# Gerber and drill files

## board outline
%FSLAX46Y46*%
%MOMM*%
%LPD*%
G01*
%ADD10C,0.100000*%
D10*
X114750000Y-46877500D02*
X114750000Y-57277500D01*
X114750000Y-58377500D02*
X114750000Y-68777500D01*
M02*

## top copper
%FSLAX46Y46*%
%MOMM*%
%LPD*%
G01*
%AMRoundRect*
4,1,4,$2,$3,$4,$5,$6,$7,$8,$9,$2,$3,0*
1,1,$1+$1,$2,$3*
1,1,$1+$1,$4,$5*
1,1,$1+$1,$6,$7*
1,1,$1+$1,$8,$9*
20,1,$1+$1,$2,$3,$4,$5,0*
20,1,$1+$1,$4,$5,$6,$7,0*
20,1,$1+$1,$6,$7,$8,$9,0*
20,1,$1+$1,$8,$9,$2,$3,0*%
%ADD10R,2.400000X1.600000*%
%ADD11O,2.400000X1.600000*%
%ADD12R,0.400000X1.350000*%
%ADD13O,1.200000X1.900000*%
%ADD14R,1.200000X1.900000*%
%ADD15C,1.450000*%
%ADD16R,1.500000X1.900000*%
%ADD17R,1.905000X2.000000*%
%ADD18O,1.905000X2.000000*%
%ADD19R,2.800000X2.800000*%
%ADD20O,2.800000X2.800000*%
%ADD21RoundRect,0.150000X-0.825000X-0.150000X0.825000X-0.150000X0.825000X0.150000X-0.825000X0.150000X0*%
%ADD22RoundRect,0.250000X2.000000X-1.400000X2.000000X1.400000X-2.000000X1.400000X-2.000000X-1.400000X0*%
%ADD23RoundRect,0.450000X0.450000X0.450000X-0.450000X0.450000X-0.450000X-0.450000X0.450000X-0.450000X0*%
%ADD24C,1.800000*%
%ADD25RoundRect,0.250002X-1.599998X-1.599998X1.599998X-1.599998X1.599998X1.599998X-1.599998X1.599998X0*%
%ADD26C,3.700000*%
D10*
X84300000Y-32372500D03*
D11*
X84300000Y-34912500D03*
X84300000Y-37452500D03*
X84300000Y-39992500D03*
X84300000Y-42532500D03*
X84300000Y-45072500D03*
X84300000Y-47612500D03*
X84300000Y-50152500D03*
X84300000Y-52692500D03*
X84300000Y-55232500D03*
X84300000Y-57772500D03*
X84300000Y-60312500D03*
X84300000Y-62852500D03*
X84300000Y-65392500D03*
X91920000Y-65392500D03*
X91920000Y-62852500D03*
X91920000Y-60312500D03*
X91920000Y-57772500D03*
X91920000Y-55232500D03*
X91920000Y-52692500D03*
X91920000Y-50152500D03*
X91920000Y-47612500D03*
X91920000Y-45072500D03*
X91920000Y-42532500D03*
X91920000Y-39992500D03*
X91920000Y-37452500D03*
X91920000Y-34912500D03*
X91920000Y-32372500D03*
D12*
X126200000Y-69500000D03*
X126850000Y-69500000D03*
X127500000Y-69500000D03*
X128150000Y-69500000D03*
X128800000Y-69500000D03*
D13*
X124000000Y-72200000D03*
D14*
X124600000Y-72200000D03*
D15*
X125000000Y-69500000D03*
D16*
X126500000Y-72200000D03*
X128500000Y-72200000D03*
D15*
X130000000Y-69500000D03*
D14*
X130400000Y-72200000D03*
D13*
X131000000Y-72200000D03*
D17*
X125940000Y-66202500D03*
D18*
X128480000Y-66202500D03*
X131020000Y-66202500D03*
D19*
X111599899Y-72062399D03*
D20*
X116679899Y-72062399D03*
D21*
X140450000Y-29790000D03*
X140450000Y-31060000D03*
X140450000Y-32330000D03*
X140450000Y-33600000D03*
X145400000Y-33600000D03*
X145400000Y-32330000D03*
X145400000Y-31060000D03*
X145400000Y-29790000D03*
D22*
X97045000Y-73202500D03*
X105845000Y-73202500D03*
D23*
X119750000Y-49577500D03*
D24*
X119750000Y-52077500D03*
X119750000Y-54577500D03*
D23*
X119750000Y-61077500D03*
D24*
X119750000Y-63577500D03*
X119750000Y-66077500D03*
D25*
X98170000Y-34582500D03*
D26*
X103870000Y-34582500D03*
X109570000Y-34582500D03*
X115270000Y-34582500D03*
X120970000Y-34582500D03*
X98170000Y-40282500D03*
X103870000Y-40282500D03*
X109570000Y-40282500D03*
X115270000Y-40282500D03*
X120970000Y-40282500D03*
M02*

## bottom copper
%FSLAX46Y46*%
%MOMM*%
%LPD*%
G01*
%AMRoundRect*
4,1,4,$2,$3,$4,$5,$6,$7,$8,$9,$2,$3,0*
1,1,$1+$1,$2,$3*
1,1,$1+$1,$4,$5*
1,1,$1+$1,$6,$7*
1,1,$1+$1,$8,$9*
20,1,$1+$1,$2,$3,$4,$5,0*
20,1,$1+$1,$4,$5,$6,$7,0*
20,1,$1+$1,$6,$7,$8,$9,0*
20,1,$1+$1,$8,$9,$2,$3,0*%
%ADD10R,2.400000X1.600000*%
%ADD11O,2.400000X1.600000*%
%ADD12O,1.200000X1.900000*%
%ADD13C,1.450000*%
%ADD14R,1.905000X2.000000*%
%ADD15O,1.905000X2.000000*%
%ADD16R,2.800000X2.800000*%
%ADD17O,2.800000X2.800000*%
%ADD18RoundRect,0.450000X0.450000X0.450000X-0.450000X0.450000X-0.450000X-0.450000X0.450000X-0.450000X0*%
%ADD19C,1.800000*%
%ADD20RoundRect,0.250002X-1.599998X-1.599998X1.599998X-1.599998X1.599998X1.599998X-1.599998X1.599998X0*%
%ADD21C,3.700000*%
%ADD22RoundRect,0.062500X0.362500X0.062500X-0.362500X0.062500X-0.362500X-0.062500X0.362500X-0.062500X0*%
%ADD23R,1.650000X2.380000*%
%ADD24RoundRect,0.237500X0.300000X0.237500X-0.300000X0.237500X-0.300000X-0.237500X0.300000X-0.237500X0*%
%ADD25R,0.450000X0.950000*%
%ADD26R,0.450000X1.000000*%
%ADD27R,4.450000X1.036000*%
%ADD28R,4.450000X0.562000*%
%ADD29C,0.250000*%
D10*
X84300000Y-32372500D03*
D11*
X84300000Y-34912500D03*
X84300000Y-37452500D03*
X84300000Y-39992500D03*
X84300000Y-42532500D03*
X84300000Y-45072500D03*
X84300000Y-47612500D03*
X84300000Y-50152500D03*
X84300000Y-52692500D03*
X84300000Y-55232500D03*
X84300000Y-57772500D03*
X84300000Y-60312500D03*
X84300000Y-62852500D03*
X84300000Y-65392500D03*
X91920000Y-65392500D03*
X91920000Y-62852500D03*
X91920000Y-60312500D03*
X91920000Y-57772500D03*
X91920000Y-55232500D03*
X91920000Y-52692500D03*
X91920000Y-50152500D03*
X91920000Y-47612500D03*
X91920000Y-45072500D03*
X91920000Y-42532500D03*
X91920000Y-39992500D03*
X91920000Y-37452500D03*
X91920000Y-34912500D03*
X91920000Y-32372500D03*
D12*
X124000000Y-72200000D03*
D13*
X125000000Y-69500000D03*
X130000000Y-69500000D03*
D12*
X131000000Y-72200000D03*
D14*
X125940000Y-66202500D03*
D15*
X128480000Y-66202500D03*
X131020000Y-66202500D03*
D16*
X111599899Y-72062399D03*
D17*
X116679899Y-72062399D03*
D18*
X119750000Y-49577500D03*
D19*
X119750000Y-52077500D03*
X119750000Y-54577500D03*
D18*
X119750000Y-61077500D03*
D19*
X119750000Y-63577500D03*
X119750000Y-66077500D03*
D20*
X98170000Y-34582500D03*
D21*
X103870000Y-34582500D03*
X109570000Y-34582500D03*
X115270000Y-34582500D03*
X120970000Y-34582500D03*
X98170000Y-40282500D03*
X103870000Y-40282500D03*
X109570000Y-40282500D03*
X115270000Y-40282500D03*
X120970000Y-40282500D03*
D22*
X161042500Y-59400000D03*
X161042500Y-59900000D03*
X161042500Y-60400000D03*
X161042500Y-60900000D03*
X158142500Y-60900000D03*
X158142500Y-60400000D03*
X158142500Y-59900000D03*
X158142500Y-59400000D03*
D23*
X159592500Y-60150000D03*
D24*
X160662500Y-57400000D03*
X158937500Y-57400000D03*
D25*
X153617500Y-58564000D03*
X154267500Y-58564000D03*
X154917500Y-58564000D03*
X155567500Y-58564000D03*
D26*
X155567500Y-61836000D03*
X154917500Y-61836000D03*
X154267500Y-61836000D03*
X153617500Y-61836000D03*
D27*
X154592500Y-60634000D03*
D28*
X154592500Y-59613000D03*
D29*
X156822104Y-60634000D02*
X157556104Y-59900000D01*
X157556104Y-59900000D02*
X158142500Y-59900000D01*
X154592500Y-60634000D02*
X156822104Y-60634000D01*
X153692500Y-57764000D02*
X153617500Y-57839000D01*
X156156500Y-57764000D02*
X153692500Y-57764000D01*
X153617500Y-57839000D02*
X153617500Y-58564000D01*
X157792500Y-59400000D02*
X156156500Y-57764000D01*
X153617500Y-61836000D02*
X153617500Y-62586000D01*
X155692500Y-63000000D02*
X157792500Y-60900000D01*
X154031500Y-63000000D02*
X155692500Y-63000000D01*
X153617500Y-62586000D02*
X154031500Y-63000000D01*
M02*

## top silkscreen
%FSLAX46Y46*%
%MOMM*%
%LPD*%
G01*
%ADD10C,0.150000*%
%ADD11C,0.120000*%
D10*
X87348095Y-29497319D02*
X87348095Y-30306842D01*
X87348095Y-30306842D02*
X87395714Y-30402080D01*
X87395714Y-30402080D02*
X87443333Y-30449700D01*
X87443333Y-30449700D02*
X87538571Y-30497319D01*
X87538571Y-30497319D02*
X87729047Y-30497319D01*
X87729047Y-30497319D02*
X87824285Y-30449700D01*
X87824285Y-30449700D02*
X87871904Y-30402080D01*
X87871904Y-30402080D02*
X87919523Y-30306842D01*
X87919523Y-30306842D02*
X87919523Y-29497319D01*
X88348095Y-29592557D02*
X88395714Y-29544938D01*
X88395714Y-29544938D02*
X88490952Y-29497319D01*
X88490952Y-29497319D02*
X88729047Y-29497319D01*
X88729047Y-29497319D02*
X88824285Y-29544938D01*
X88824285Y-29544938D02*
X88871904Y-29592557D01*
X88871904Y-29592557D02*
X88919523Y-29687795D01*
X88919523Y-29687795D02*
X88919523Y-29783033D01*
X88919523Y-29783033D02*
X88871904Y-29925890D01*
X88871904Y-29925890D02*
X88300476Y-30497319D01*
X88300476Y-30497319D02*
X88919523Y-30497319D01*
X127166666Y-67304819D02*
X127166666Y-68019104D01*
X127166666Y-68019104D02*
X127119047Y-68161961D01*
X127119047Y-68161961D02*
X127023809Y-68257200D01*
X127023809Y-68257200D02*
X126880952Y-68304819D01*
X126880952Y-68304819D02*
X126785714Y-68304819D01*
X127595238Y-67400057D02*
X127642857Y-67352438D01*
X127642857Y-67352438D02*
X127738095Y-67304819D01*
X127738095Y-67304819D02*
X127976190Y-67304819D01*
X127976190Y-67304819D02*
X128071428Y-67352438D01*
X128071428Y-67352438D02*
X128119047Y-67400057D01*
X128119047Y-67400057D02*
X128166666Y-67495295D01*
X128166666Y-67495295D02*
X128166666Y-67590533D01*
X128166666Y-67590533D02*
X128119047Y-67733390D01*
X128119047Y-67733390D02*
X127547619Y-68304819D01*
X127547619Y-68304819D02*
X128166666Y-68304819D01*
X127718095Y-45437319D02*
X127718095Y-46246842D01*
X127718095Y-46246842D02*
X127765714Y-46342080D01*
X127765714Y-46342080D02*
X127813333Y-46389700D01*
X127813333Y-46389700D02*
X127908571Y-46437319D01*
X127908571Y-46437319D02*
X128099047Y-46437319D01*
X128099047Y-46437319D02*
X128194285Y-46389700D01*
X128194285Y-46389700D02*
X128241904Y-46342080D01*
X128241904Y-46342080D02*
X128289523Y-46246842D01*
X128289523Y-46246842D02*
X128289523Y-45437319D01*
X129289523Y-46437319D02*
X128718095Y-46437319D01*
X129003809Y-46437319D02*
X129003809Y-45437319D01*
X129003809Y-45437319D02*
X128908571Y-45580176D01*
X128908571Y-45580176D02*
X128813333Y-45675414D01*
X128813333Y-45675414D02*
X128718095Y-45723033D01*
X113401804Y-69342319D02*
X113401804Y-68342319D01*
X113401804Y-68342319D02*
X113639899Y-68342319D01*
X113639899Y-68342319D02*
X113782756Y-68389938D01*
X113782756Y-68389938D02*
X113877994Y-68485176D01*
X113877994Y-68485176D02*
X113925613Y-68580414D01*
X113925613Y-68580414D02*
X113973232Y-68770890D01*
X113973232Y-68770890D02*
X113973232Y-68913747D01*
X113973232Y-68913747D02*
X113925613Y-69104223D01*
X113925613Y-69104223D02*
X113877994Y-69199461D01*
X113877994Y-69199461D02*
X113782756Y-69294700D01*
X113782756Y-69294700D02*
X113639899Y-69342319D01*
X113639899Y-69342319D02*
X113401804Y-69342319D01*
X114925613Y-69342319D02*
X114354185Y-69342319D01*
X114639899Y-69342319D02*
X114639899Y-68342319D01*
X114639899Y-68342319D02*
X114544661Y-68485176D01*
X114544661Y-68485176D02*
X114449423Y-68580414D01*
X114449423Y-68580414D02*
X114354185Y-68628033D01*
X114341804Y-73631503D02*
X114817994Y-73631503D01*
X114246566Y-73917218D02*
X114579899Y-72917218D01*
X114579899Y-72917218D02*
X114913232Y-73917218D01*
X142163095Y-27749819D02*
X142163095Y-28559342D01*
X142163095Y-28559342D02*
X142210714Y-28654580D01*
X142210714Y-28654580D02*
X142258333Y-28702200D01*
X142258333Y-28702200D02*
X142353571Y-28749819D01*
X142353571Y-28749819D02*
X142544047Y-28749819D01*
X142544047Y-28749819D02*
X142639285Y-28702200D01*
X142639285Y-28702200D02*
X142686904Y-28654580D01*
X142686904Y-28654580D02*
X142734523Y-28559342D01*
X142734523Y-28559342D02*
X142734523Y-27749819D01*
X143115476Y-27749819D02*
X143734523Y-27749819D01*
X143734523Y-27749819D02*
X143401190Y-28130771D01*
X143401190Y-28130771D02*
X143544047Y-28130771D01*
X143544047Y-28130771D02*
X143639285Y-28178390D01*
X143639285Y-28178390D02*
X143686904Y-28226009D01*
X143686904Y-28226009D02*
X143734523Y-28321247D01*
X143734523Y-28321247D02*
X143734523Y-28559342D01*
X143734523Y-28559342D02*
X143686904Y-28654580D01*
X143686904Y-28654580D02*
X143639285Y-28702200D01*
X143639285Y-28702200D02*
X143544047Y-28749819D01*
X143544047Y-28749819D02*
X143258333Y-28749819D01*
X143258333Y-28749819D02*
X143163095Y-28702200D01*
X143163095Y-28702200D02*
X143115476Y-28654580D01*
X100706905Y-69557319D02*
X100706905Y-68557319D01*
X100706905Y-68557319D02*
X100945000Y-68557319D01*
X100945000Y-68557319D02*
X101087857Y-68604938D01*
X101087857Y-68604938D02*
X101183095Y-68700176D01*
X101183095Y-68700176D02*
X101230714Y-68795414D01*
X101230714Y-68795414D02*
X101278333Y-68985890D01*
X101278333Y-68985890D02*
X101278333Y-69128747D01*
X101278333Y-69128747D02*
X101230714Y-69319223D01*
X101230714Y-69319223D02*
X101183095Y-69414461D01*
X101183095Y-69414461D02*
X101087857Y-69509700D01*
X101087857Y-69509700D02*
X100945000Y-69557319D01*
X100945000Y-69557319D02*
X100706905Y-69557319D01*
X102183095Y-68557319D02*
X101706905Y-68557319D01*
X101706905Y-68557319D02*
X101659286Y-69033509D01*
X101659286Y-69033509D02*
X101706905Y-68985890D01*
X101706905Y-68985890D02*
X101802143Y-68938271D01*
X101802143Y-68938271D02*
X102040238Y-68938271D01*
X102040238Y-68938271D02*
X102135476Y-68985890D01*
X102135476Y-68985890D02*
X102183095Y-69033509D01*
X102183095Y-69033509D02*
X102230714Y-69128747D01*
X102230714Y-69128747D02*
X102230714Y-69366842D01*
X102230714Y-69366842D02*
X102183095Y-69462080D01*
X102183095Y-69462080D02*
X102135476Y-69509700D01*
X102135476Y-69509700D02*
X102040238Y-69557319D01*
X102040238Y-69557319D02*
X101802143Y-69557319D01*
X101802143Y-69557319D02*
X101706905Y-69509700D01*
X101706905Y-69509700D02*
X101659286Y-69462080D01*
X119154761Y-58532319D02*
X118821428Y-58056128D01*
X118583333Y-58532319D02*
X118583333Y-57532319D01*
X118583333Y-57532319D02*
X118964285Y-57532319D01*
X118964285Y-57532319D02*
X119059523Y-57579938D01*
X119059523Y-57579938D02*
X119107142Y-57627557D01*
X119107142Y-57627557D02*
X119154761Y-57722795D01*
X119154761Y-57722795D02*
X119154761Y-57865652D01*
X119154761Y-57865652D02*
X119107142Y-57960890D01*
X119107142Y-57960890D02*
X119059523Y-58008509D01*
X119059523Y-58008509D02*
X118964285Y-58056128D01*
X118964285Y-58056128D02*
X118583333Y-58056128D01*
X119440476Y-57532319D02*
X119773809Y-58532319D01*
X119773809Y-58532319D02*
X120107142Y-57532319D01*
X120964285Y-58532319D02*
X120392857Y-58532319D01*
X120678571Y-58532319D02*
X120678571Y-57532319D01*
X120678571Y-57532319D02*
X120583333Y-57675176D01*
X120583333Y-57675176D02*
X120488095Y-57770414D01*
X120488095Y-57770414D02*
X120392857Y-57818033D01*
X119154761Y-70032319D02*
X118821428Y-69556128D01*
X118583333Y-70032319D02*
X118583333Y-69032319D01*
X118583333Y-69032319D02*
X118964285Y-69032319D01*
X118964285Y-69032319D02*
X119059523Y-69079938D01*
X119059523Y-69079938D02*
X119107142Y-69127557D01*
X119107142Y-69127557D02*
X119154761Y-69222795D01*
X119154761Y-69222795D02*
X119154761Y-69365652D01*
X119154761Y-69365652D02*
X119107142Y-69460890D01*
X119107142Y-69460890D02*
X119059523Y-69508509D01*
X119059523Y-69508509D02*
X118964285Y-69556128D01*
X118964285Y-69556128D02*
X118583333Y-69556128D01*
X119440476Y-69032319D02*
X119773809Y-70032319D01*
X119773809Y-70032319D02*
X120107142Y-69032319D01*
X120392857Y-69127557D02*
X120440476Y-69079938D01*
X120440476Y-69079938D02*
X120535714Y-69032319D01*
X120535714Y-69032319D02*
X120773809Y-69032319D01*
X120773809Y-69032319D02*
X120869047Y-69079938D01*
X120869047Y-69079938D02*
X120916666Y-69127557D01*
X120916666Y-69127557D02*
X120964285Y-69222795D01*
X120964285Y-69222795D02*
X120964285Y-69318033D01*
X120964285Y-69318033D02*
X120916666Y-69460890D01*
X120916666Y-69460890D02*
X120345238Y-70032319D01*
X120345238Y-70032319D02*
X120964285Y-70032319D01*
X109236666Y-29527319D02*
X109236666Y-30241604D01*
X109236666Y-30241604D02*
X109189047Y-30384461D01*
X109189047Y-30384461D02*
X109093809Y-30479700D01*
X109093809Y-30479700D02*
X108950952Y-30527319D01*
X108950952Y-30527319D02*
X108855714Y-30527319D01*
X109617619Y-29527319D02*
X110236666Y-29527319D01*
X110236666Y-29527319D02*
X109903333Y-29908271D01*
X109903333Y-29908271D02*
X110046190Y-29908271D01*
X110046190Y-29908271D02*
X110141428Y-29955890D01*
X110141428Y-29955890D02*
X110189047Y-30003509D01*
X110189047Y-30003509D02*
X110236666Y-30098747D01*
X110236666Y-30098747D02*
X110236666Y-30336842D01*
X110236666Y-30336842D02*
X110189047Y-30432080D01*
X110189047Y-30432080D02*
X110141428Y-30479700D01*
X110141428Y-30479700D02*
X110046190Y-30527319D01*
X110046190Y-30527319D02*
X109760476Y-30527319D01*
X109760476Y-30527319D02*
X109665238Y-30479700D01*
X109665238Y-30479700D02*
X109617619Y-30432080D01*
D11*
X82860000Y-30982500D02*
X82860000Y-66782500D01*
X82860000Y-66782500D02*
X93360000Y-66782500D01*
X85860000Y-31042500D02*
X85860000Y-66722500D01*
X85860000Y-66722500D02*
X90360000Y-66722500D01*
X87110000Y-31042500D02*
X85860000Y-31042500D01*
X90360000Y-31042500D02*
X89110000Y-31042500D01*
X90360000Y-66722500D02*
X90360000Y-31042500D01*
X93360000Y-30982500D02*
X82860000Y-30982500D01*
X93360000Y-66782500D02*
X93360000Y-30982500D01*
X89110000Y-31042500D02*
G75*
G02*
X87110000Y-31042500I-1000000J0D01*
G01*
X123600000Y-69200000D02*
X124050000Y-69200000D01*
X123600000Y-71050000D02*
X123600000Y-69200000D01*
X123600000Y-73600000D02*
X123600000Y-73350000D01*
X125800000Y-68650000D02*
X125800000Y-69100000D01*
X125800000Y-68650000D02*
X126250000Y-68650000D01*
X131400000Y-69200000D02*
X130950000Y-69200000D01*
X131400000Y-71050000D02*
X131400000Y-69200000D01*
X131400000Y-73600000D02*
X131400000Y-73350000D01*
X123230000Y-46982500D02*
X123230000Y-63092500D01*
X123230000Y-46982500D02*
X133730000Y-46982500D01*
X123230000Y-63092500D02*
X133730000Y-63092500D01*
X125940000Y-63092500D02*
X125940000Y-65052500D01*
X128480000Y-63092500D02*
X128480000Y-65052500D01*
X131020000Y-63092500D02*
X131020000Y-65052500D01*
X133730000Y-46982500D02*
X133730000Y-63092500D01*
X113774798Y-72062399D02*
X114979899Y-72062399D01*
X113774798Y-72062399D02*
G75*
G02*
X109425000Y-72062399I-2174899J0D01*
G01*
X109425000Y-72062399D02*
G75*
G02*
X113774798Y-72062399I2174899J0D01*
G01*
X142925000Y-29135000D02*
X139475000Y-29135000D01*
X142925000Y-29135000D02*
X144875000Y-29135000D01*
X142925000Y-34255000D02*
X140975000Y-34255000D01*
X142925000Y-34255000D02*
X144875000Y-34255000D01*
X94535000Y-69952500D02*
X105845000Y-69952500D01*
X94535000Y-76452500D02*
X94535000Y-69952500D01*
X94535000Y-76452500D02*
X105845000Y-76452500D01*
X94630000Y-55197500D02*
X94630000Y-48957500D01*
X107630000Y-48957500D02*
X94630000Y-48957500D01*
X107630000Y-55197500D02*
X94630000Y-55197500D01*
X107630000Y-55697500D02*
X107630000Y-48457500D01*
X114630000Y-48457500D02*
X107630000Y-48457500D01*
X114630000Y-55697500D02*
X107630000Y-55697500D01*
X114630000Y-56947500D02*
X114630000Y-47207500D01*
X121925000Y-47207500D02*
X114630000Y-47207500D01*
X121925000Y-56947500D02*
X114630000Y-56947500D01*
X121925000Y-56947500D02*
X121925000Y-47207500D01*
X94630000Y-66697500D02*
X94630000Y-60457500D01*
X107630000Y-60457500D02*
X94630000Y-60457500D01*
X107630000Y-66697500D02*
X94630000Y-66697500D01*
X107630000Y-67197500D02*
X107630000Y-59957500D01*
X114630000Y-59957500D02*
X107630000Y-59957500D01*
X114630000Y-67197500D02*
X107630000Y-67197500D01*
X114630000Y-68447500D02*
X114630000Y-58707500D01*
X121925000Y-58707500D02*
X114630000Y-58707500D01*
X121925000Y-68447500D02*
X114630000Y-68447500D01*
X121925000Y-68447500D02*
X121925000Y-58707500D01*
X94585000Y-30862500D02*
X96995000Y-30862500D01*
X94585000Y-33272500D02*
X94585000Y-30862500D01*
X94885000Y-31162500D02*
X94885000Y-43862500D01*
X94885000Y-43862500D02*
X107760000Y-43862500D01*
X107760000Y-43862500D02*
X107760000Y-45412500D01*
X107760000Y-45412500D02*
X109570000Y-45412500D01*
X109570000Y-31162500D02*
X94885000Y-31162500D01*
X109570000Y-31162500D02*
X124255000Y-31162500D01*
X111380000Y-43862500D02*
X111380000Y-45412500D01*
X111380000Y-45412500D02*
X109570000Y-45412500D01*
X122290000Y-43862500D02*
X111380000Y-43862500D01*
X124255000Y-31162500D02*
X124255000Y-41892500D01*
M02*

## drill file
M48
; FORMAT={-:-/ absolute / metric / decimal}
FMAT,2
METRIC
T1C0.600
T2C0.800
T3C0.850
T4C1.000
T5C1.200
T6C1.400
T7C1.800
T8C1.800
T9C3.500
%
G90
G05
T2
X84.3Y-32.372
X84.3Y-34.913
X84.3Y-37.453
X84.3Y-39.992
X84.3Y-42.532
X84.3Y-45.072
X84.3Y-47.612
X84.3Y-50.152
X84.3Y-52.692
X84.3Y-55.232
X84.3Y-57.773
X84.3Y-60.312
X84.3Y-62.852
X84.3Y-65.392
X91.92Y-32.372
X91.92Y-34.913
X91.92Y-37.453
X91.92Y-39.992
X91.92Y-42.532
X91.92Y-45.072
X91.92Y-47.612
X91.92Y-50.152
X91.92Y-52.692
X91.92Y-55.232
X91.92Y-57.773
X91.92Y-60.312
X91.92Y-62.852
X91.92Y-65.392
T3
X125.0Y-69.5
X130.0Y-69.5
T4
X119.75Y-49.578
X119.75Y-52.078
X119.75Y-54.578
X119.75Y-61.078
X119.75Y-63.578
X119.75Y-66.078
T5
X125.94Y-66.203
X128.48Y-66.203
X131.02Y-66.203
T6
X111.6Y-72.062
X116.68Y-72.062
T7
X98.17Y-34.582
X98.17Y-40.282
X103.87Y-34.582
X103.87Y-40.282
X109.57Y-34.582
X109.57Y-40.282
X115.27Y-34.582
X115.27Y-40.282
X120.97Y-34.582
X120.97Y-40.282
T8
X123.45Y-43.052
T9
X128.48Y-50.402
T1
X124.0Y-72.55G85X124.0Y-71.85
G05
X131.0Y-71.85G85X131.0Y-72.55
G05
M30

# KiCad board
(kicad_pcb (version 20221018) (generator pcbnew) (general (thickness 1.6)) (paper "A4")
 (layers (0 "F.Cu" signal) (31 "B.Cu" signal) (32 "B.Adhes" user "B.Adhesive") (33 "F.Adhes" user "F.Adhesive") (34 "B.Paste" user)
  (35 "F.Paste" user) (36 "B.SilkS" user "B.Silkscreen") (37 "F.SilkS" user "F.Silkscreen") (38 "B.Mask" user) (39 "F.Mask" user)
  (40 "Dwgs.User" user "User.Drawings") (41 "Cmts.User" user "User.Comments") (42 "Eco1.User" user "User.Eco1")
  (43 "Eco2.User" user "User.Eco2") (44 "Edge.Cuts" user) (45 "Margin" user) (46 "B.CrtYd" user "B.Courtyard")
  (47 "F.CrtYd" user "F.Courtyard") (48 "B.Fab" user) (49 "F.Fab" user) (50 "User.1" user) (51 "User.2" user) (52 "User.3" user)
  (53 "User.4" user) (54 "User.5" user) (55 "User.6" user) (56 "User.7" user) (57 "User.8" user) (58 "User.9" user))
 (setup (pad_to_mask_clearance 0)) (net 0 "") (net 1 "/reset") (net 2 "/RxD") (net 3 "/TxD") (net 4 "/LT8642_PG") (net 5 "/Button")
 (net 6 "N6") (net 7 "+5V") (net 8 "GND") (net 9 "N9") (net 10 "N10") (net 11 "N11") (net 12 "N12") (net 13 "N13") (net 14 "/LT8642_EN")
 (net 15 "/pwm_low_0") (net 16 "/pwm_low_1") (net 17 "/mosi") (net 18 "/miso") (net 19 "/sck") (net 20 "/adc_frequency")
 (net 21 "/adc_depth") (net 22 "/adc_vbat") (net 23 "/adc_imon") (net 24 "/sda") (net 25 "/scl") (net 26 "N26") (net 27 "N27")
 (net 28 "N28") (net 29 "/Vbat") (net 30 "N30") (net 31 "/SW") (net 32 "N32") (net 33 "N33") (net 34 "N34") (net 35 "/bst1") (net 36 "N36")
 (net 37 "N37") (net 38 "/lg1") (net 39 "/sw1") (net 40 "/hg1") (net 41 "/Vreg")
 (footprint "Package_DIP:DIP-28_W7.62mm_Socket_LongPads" (layer "F.Cu") (at 84.3 32.3725)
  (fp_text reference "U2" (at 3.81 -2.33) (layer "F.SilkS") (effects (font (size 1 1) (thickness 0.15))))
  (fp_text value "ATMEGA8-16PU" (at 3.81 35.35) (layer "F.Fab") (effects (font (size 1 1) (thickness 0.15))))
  (fp_line (start -1.44 -1.39) (end -1.44 34.41) (stroke (width 0.12) (type solid)) (layer "F.SilkS"))
  (fp_line (start -1.44 34.41) (end 9.06 34.41) (stroke (width 0.12) (type solid)) (layer "F.SilkS"))
  (fp_line (start 1.56 -1.33) (end 1.56 34.35) (stroke (width 0.12) (type solid)) (layer "F.SilkS"))
  (fp_line (start 1.56 34.35) (end 6.06 34.35) (stroke (width 0.12) (type solid)) (layer "F.SilkS"))
  (fp_line (start 2.81 -1.33) (end 1.56 -1.33) (stroke (width 0.12) (type solid)) (layer "F.SilkS"))
  (fp_line (start 6.06 -1.33) (end 4.81 -1.33) (stroke (width 0.12) (type solid)) (layer "F.SilkS"))
  (fp_line (start 6.06 34.35) (end 6.06 -1.33) (stroke (width 0.12) (type solid)) (layer "F.SilkS"))
  (fp_line (start 9.06 -1.39) (end -1.44 -1.39) (stroke (width 0.12) (type solid)) (layer "F.SilkS"))
  (fp_line (start 9.06 34.41) (end 9.06 -1.39) (stroke (width 0.12) (type solid)) (layer "F.SilkS"))
  (fp_arc (start 4.81 -1.33) (mid 3.81 -0.33) (end 2.81 -1.33) (stroke (width 0.12) (type solid)) (layer "F.SilkS"))
  (pad "1" thru_hole rect (at 0 0) (size 2.4 1.6) (drill 0.8) (layers "*.Cu" "*.Mask") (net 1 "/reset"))
  (pad "2" thru_hole oval (at 0 2.54) (size 2.4 1.6) (drill 0.8) (layers "*.Cu" "*.Mask") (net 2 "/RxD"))
  (pad "3" thru_hole oval (at 0 5.08) (size 2.4 1.6) (drill 0.8) (layers "*.Cu" "*.Mask") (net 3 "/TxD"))
  (pad "4" thru_hole oval (at 0 7.62) (size 2.4 1.6) (drill 0.8) (layers "*.Cu" "*.Mask") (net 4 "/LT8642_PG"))
  (pad "5" thru_hole oval (at 0 10.16) (size 2.4 1.6) (drill 0.8) (layers "*.Cu" "*.Mask") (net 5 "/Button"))
  (pad "6" thru_hole oval (at 0 12.7) (size 2.4 1.6) (drill 0.8) (layers "*.Cu" "*.Mask") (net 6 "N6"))
  (pad "7" thru_hole oval (at 0 15.24) (size 2.4 1.6) (drill 0.8) (layers "*.Cu" "*.Mask") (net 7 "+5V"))
  (pad "8" thru_hole oval (at 0 17.78) (size 2.4 1.6) (drill 0.8) (layers "*.Cu" "*.Mask") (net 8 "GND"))
  (pad "9" thru_hole oval (at 0 20.32) (size 2.4 1.6) (drill 0.8) (layers "*.Cu" "*.Mask") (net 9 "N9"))
  (pad "10" thru_hole oval (at 0 22.86) (size 2.4 1.6) (drill 0.8) (layers "*.Cu" "*.Mask") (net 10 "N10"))
  (pad "11" thru_hole oval (at 0 25.4) (size 2.4 1.6) (drill 0.8) (layers "*.Cu" "*.Mask") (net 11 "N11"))
  (pad "12" thru_hole oval (at 0 27.94) (size 2.4 1.6) (drill 0.8) (layers "*.Cu" "*.Mask") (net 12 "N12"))
  (pad "13" thru_hole oval (at 0 30.48) (size 2.4 1.6) (drill 0.8) (layers "*.Cu" "*.Mask") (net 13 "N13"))
  (pad "14" thru_hole oval (at 0 33.02) (size 2.4 1.6) (drill 0.8) (layers "*.Cu" "*.Mask") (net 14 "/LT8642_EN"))
  (pad "15" thru_hole oval (at 7.62 33.02) (size 2.4 1.6) (drill 0.8) (layers "*.Cu" "*.Mask") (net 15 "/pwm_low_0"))
  (pad "16" thru_hole oval (at 7.62 30.48) (size 2.4 1.6) (drill 0.8) (layers "*.Cu" "*.Mask") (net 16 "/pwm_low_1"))
  (pad "17" thru_hole oval (at 7.62 27.94) (size 2.4 1.6) (drill 0.8) (layers "*.Cu" "*.Mask") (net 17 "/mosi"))
  (pad "18" thru_hole oval (at 7.62 25.4) (size 2.4 1.6) (drill 0.8) (layers "*.Cu" "*.Mask") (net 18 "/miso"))
  (pad "19" thru_hole oval (at 7.62 22.86) (size 2.4 1.6) (drill 0.8) (layers "*.Cu" "*.Mask") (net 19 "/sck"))
  (pad "20" thru_hole oval (at 7.62 20.32) (size 2.4 1.6) (drill 0.8) (layers "*.Cu" "*.Mask") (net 7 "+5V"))
  (pad "21" thru_hole oval (at 7.62 17.78) (size 2.4 1.6) (drill 0.8) (layers "*.Cu" "*.Mask") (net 7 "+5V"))
  (pad "22" thru_hole oval (at 7.62 15.24) (size 2.4 1.6) (drill 0.8) (layers "*.Cu" "*.Mask") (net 8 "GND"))
  (pad "23" thru_hole oval (at 7.62 12.7) (size 2.4 1.6) (drill 0.8) (layers "*.Cu" "*.Mask") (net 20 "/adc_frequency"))
  (pad "24" thru_hole oval (at 7.62 10.16) (size 2.4 1.6) (drill 0.8) (layers "*.Cu" "*.Mask") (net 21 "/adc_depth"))
  (pad "25" thru_hole oval (at 7.62 7.62) (size 2.4 1.6) (drill 0.8) (layers "*.Cu" "*.Mask") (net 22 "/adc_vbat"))
  (pad "26" thru_hole oval (at 7.62 5.08) (size 2.4 1.6) (drill 0.8) (layers "*.Cu" "*.Mask") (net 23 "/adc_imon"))
  (pad "27" thru_hole oval (at 7.62 2.54) (size 2.4 1.6) (drill 0.8) (layers "*.Cu" "*.Mask") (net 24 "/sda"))
  (pad "28" thru_hole oval (at 7.62 0) (size 2.4 1.6) (drill 0.8) (layers "*.Cu" "*.Mask") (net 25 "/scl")))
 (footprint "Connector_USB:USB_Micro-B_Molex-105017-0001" (layer "F.Cu") (at 127.5 70.9625)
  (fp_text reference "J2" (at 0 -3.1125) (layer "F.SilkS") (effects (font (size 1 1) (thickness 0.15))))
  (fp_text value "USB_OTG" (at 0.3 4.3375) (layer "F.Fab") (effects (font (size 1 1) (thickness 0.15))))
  (fp_line (start -3.9 -1.7625) (end -3.45 -1.7625) (stroke (width 0.12) (type solid)) (layer "F.SilkS"))
  (fp_line (start -3.9 0.0875) (end -3.9 -1.7625) (stroke (width 0.12) (type solid)) (layer "F.SilkS"))
  (fp_line (start -3.9 2.6375) (end -3.9 2.3875) (stroke (width 0.12) (type solid)) (layer "F.SilkS"))
  (fp_line (start -1.7 -2.3125) (end -1.7 -1.8625) (stroke (width 0.12) (type solid)) (layer "F.SilkS"))
  (fp_line (start -1.7 -2.3125) (end -1.25 -2.3125) (stroke (width 0.12) (type solid)) (layer "F.SilkS"))
  (fp_line (start 3.9 -1.7625) (end 3.45 -1.7625) (stroke (width 0.12) (type solid)) (layer "F.SilkS"))
  (fp_line (start 3.9 0.0875) (end 3.9 -1.7625) (stroke (width 0.12) (type solid)) (layer "F.SilkS"))
  (fp_line (start 3.9 2.6375) (end 3.9 2.3875) (stroke (width 0.12) (type solid)) (layer "F.SilkS"))
  (pad "1" smd rect (at -1.3 -1.4625) (size 0.4 1.35) (layers "F.Cu" "F.Paste" "F.Mask") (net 7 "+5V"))
  (pad "2" smd rect (at -0.65 -1.4625) (size 0.4 1.35) (layers "F.Cu" "F.Paste" "F.Mask") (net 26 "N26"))
  (pad "3" smd rect (at 0 -1.4625) (size 0.4 1.35) (layers "F.Cu" "F.Paste" "F.Mask") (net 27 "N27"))
  (pad "4" smd rect (at 0.65 -1.4625) (size 0.4 1.35) (layers "F.Cu" "F.Paste" "F.Mask") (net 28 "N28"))
  (pad "5" smd rect (at 1.3 -1.4625) (size 0.4 1.35) (layers "F.Cu" "F.Paste" "F.Mask") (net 8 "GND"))
  (pad "6" thru_hole oval (at -3.5 1.2375 180) (size 1.2 1.9) (drill oval 0.6 1.3) (layers "*.Cu" "*.Mask") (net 8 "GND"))
  (pad "6" smd rect (at -2.9 1.2375) (size 1.2 1.9) (layers "F.Cu" "F.Mask") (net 8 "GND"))
  (pad "6" thru_hole circle (at -2.5 -1.4625) (size 1.45 1.45) (drill 0.85) (layers "*.Cu" "*.Mask") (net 8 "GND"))
  (pad "6" smd rect (at -1 1.2375) (size 1.5 1.9) (layers "F.Cu" "F.Paste" "F.Mask") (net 8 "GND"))
  (pad "6" smd rect (at 1 1.2375) (size 1.5 1.9) (layers "F.Cu" "F.Paste" "F.Mask") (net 8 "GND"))
  (pad "6" thru_hole circle (at 2.5 -1.4625) (size 1.45 1.45) (drill 0.85) (layers "*.Cu" "*.Mask") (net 8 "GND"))
  (pad "6" smd rect (at 2.9 1.2375) (size 1.2 1.9) (layers "F.Cu" "F.Mask") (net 8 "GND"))
  (pad "6" thru_hole oval (at 3.5 1.2375) (size 1.2 1.9) (drill oval 0.6 1.3) (layers "*.Cu" "*.Mask") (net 8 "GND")))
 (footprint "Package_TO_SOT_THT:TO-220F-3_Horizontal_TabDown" (layer "F.Cu") (at 125.94 66.2025)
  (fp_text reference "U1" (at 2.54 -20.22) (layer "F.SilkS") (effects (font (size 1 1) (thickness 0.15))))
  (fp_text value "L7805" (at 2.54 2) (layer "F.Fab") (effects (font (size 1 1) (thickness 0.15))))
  (fp_line (start -2.71 -19.22) (end -2.71 -3.11) (stroke (width 0.12) (type solid)) (layer "F.SilkS"))
  (fp_line (start -2.71 -19.22) (end 7.79 -19.22) (stroke (width 0.12) (type solid)) (layer "F.SilkS"))
  (fp_line (start -2.71 -3.11) (end 7.79 -3.11) (stroke (width 0.12) (type solid)) (layer "F.SilkS"))
  (fp_line (start 0 -3.11) (end 0 -1.15) (stroke (width 0.12) (type solid)) (layer "F.SilkS"))
  (fp_line (start 2.54 -3.11) (end 2.54 -1.15) (stroke (width 0.12) (type solid)) (layer "F.SilkS"))
  (fp_line (start 5.08 -3.11) (end 5.08 -1.15) (stroke (width 0.12) (type solid)) (layer "F.SilkS"))
  (fp_line (start 7.79 -19.22) (end 7.79 -3.11) (stroke (width 0.12) (type solid)) (layer "F.SilkS"))
  (pad "" np_thru_hole oval (at 2.54 -15.8) (size 3.5 3.5) (drill 3.5) (layers "*.Cu" "*.Mask"))
  (pad "1" thru_hole rect (at 0 0) (size 1.905 2) (drill 1.2) (layers "*.Cu" "*.Mask") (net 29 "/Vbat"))
  (pad "2" thru_hole oval (at 2.54 0) (size 1.905 2) (drill 1.2) (layers "*.Cu" "*.Mask") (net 8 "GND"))
  (pad "3" thru_hole oval (at 5.08 0) (size 1.905 2) (drill 1.2) (layers "*.Cu" "*.Mask") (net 7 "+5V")))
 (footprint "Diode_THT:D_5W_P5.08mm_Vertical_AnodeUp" (layer "F.Cu") (at 111.599899 72.062399)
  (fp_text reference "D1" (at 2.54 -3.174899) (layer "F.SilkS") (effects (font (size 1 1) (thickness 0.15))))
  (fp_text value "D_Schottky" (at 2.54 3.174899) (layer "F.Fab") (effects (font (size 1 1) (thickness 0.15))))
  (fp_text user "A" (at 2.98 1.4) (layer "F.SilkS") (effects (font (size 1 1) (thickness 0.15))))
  (fp_line (start 2.174899 0) (end 3.38 0) (stroke (width 0.12) (type solid)) (layer "F.SilkS"))
  (fp_circle (center 0 0) (end 2.174899 0) (stroke (width 0.12) (type solid)) (fill none) (layer "F.SilkS"))
  (pad "1" thru_hole rect (at 0 0) (size 2.8 2.8) (drill 1.4) (layers "*.Cu" "*.Mask") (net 29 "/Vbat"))
  (pad "2" thru_hole oval (at 5.08 0) (size 2.8 2.8) (drill 1.4) (layers "*.Cu" "*.Mask") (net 7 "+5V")))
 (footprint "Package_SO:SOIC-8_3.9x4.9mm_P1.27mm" (layer "F.Cu") (at 142.925 31.695)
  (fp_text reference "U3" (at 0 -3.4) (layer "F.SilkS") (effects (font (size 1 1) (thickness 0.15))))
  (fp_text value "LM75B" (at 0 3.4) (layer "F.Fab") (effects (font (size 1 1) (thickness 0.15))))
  (fp_line (start 0 -2.56) (end -3.45 -2.56) (stroke (width 0.12) (type solid)) (layer "F.SilkS"))
  (fp_line (start 0 -2.56) (end 1.95 -2.56) (stroke (width 0.12) (type solid)) (layer "F.SilkS"))
  (fp_line (start 0 2.56) (end -1.95 2.56) (stroke (width 0.12) (type solid)) (layer "F.SilkS"))
  (fp_line (start 0 2.56) (end 1.95 2.56) (stroke (width 0.12) (type solid)) (layer "F.SilkS"))
  (pad "1" smd roundrect (at -2.475 -1.905) (size 1.95 0.6) (layers "F.Cu" "F.Paste" "F.Mask") (roundrect_rratio 0.25) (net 24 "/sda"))
  (pad "2" smd roundrect (at -2.475 -0.635) (size 1.95 0.6) (layers "F.Cu" "F.Paste" "F.Mask") (roundrect_rratio 0.25) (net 25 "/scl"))
  (pad "3" smd roundrect (at -2.475 0.635) (size 1.95 0.6) (layers "F.Cu" "F.Paste" "F.Mask") (roundrect_rratio 0.25) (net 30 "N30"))
  (pad "4" smd roundrect (at -2.475 1.905) (size 1.95 0.6) (layers "F.Cu" "F.Paste" "F.Mask") (roundrect_rratio 0.25) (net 8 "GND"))
  (pad "5" smd roundrect (at 2.475 1.905) (size 1.95 0.6) (layers "F.Cu" "F.Paste" "F.Mask") (roundrect_rratio 0.25) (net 8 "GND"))
  (pad "6" smd roundrect (at 2.475 0.635) (size 1.95 0.6) (layers "F.Cu" "F.Paste" "F.Mask") (roundrect_rratio 0.25) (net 8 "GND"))
  (pad "7" smd roundrect (at 2.475 -0.635) (size 1.95 0.6) (layers "F.Cu" "F.Paste" "F.Mask") (roundrect_rratio 0.25) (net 7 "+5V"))
  (pad "8" smd roundrect (at 2.475 -1.905) (size 1.95 0.6) (layers "F.Cu" "F.Paste" "F.Mask") (roundrect_rratio 0.25) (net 7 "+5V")))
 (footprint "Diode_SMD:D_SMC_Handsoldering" (layer "F.Cu") (at 101.445 73.2025)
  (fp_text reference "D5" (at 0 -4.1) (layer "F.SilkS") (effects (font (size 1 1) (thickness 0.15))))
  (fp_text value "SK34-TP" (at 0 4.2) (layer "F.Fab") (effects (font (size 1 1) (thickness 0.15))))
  (fp_line (start -6.91 -3.25) (end 4.4 -3.25) (stroke (width 0.12) (type solid)) (layer "F.SilkS"))
  (fp_line (start -6.91 3.25) (end -6.91 -3.25) (stroke (width 0.12) (type solid)) (layer "F.SilkS"))
  (fp_line (start -6.91 3.25) (end 4.4 3.25) (stroke (width 0.12) (type solid)) (layer "F.SilkS"))
  (pad "1" smd roundrect (at -4.4 0 90) (size 3.3 4.5) (layers "F.Cu" "F.Paste" "F.Mask") (roundrect_rratio 0.0757575758) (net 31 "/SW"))
  (pad "2" smd roundrect (at 4.4 0 90) (size 3.3 4.5) (layers "F.Cu" "F.Paste" "F.Mask") (roundrect_rratio 0.0757575758) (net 8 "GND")))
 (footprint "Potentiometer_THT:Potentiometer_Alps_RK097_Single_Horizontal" (layer "F.Cu") (at 119.75 49.5775)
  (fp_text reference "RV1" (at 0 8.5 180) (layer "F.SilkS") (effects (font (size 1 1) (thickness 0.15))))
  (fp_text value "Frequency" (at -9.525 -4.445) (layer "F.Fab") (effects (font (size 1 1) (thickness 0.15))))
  (fp_line (start -25.12 5.62) (end -25.12 -0.62) (stroke (width 0.12) (type solid)) (layer "F.SilkS"))
  (fp_line (start -12.12 -0.62) (end -25.12 -0.62) (stroke (width 0.12) (type solid)) (layer "F.SilkS"))
  (fp_line (start -12.12 5.62) (end -25.12 5.62) (stroke (width 0.12) (type solid)) (layer "F.SilkS"))
  (fp_line (start -12.12 6.12) (end -12.12 -1.12) (stroke (width 0.12) (type solid)) (layer "F.SilkS"))
  (fp_line (start -5.12 -1.12) (end -12.12 -1.12) (stroke (width 0.12) (type solid)) (layer "F.SilkS"))
  (fp_line (start -5.12 6.12) (end -12.12 6.12) (stroke (width 0.12) (type solid)) (layer "F.SilkS"))
  (fp_line (start -5.12 7.37) (end -5.12 -2.37) (stroke (width 0.12) (type solid)) (layer "F.SilkS"))
  (fp_line (start 2.175 -2.37) (end -5.12 -2.37) (stroke (width 0.12) (type solid)) (layer "F.SilkS"))
  (fp_line (start 2.175 7.37) (end -5.12 7.37) (stroke (width 0.12) (type solid)) (layer "F.SilkS"))
  (fp_line (start 2.175 7.37) (end 2.175 -2.37) (stroke (width 0.12) (type solid)) (layer "F.SilkS"))
  (fp_line (start -5 -2.7) (end -5 7.7) (stroke (width 0.1) (type solid)) (layer "Edge.Cuts"))
  (pad "1" thru_hole roundrect (at 0 0 180) (size 1.8 1.8) (drill 1) (layers "*.Cu" "*.Mask") (roundrect_rratio 0.25) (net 7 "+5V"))
  (pad "2" thru_hole circle (at 0 2.5 180) (size 1.8 1.8) (drill 1) (layers "*.Cu" "*.Mask") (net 20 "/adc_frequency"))
  (pad "3" thru_hole circle (at 0 5 180) (size 1.8 1.8) (drill 1) (layers "*.Cu" "*.Mask") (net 8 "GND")))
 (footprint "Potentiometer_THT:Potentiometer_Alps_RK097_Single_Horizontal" (layer "F.Cu") (at 119.75 61.0775)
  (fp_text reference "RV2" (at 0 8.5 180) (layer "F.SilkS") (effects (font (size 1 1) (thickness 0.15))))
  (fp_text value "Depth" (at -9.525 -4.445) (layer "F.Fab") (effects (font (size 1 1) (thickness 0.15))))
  (fp_line (start -25.12 5.62) (end -25.12 -0.62) (stroke (width 0.12) (type solid)) (layer "F.SilkS"))
  (fp_line (start -12.12 -0.62) (end -25.12 -0.62) (stroke (width 0.12) (type solid)) (layer "F.SilkS"))
  (fp_line (start -12.12 5.62) (end -25.12 5.62) (stroke (width 0.12) (type solid)) (layer "F.SilkS"))
  (fp_line (start -12.12 6.12) (end -12.12 -1.12) (stroke (width 0.12) (type solid)) (layer "F.SilkS"))
  (fp_line (start -5.12 -1.12) (end -12.12 -1.12) (stroke (width 0.12) (type solid)) (layer "F.SilkS"))
  (fp_line (start -5.12 6.12) (end -12.12 6.12) (stroke (width 0.12) (type solid)) (layer "F.SilkS"))
  (fp_line (start -5.12 7.37) (end -5.12 -2.37) (stroke (width 0.12) (type solid)) (layer "F.SilkS"))
  (fp_line (start 2.175 -2.37) (end -5.12 -2.37) (stroke (width 0.12) (type solid)) (layer "F.SilkS"))
  (fp_line (start 2.175 7.37) (end -5.12 7.37) (stroke (width 0.12) (type solid)) (layer "F.SilkS"))
  (fp_line (start 2.175 7.37) (end 2.175 -2.37) (stroke (width 0.12) (type solid)) (layer "F.SilkS"))
  (fp_line (start -5 -2.7) (end -5 7.7) (stroke (width 0.1) (type solid)) (layer "Edge.Cuts"))
  (pad "1" thru_hole roundrect (at 0 0 180) (size 1.8 1.8) (drill 1) (layers "*.Cu" "*.Mask") (roundrect_rratio 0.25) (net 7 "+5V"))
  (pad "2" thru_hole circle (at 0 2.5 180) (size 1.8 1.8) (drill 1) (layers "*.Cu" "*.Mask") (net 21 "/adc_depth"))
  (pad "3" thru_hole circle (at 0 5 180) (size 1.8 1.8) (drill 1) (layers "*.Cu" "*.Mask") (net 8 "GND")))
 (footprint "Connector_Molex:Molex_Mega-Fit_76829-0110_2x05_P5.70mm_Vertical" (layer "F.Cu") (at 98.17 34.5825)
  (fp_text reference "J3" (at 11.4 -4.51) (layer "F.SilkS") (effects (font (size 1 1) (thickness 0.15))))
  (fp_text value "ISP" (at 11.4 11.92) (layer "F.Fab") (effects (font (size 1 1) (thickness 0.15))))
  (fp_line (start -3.585 -3.72) (end -1.175 -3.72) (stroke (width 0.12) (type solid)) (layer "F.SilkS"))
  (fp_line (start -3.585 -1.31) (end -3.585 -3.72) (stroke (width 0.12) (type solid)) (layer "F.SilkS"))
  (fp_line (start -3.285 -3.42) (end -3.285 9.28) (stroke (width 0.12) (type solid)) (layer "F.SilkS"))
  (fp_line (start -3.285 9.28) (end 9.59 9.28) (stroke (width 0.12) (type solid)) (layer "F.SilkS"))
  (fp_line (start 9.59 9.28) (end 9.59 10.83) (stroke (width 0.12) (type solid)) (layer "F.SilkS"))
  (fp_line (start 9.59 10.83) (end 11.4 10.83) (stroke (width 0.12) (type solid)) (layer "F.SilkS"))
  (fp_line (start 11.4 -3.42) (end -3.285 -3.42) (stroke (width 0.12) (type solid)) (layer "F.SilkS"))
  (fp_line (start 11.4 -3.42) (end 26.085 -3.42) (stroke (width 0.12) (type solid)) (layer "F.SilkS"))
  (fp_line (start 13.21 9.28) (end 13.21 10.83) (stroke (width 0.12) (type solid)) (layer "F.SilkS"))
  (fp_line (start 13.21 10.83) (end 11.4 10.83) (stroke (width 0.12) (type solid)) (layer "F.SilkS"))
  (fp_line (start 24.12 9.28) (end 13.21 9.28) (stroke (width 0.12) (type solid)) (layer "F.SilkS"))
  (fp_line (start 26.085 -3.42) (end 26.085 7.31) (stroke (width 0.12) (type solid)) (layer "F.SilkS"))
  (pad "" np_thru_hole circle (at 25.28 8.47) (size 1.8 1.8) (drill 1.8) (layers "*.Cu" "*.Mask"))
  (pad "1" thru_hole roundrect (at 0 0) (size 3.7 3.7) (drill 1.8) (layers "*.Cu" "*.Mask") (roundrect_rratio 0.067568) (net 17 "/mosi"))
  (pad "2" thru_hole circle (at 5.7 0) (size 3.7 3.7) (drill 1.8) (layers "*.Cu" "*.Mask") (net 7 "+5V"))
  (pad "3" thru_hole circle (at 11.4 0) (size 3.7 3.7) (drill 1.8) (layers "*.Cu" "*.Mask") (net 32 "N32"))
  (pad "4" thru_hole circle (at 17.1 0) (size 3.7 3.7) (drill 1.8) (layers "*.Cu" "*.Mask") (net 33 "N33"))
  (pad "5" thru_hole circle (at 22.8 0) (size 3.7 3.7) (drill 1.8) (layers "*.Cu" "*.Mask") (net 1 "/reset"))
  (pad "6" thru_hole circle (at 0 5.7) (size 3.7 3.7) (drill 1.8) (layers "*.Cu" "*.Mask") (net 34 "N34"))
  (pad "7" thru_hole circle (at 5.7 5.7) (size 3.7 3.7) (drill 1.8) (layers "*.Cu" "*.Mask") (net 19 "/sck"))
  (pad "8" thru_hole circle (at 11.4 5.7) (size 3.7 3.7) (drill 1.8) (layers "*.Cu" "*.Mask") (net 8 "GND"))
  (pad "9" thru_hole circle (at 17.1 5.7) (size 3.7 3.7) (drill 1.8) (layers "*.Cu" "*.Mask") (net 18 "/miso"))
  (pad "10" thru_hole circle (at 22.8 5.7) (size 3.7 3.7) (drill 1.8) (layers "*.Cu" "*.Mask") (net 8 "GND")))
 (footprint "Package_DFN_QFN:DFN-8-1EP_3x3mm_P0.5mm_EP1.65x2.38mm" (layer "B.Cu") (at 159.5925 60.15 180)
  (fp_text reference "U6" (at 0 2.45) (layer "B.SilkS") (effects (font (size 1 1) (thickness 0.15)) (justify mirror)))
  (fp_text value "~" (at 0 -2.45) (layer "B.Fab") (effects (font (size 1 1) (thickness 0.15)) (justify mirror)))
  (pad "" smd roundrect (at 0 0 180) (size 1.33 1.92) (layers "B.Paste") (roundrect_rratio 0.18797))
  (pad "1" smd roundrect (at -1.45 0.75 180) (size 0.85 0.25) (layers "B.Cu" "B.Paste" "B.Mask") (roundrect_rratio 0.25) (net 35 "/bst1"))
  (pad "2" smd roundrect (at -1.45 0.25 180) (size 0.85 0.25) (layers "B.Cu" "B.Paste" "B.Mask") (roundrect_rratio 0.25) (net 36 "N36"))
  (pad "3" smd roundrect (at -1.45 -0.25 180) (size 0.85 0.25) (layers "B.Cu" "B.Paste" "B.Mask") (roundrect_rratio 0.25) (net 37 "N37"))
  (pad "4" smd roundrect (at -1.45 -0.75 180) (size 0.85 0.25) (layers "B.Cu" "B.Paste" "B.Mask") (roundrect_rratio 0.25) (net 7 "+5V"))
  (pad "5" smd roundrect (at 1.45 -0.75 180) (size 0.85 0.25) (layers "B.Cu" "B.Paste" "B.Mask") (roundrect_rratio 0.25) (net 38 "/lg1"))
  (pad "6" smd roundrect (at 1.45 -0.25 180) (size 0.85 0.25) (layers "B.Cu" "B.Paste" "B.Mask") (roundrect_rratio 0.25) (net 8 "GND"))
  (pad "7" smd roundrect (at 1.45 0.25 180) (size 0.85 0.25) (layers "B.Cu" "B.Paste" "B.Mask") (roundrect_rratio 0.25) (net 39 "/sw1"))
  (pad "8" smd roundrect (at 1.45 0.75 180) (size 0.85 0.25) (layers "B.Cu" "B.Paste" "B.Mask") (roundrect_rratio 0.25) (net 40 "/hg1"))
  (pad "9" smd rect (at 0 0 180) (size 1.65 2.38) (layers "B.Cu" "B.Mask") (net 8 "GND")))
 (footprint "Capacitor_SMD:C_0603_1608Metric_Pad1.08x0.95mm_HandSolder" (layer "B.Cu") (at 159.8 57.4 180)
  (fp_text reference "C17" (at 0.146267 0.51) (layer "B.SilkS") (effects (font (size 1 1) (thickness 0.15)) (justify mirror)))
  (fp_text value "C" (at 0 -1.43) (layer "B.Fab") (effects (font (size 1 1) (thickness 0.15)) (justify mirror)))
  (pad "1" smd roundrect (at -0.8625 0 180) (size 1.075 0.95) (layers "B.Cu" "B.Paste" "B.Mask") (roundrect_rratio 0.25) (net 35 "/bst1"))
  (pad "2" smd roundrect (at 0.8625 0 180) (size 1.075 0.95) (layers "B.Cu" "B.Paste" "B.Mask") (roundrect_rratio 0.25) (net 39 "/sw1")))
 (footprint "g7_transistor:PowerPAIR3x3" (layer "B.Cu") (at 154.5925 60.2)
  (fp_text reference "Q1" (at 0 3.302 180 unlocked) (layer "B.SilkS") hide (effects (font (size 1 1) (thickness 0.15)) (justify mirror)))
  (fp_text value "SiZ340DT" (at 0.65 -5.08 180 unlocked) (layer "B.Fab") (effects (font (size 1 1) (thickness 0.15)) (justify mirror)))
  (pad "1" smd rect (at -0.975 -1.636) (size 0.45 0.95) (layers "B.Cu" "B.Paste" "B.Mask") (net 40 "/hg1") (thermal_bridge_angle 45))
  (pad "2" smd rect (at -0.325 -1.636) (size 0.45 0.95) (layers "B.Cu" "B.Paste" "B.Mask") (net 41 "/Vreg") (thermal_bridge_angle 45))
  (pad "3" smd rect (at 0.325 -1.636) (size 0.45 0.95) (layers "B.Cu" "B.Paste" "B.Mask") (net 41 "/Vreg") (thermal_bridge_angle 45))
  (pad "4" smd rect (at 0.975 -1.636) (size 0.45 0.95) (layers "B.Cu" "B.Paste" "B.Mask") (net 41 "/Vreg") (thermal_bridge_angle 45))
  (pad "5" smd rect (at 0.975 1.636) (size 0.45 1) (layers "B.Cu" "B.Paste" "B.Mask") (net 8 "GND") (thermal_bridge_angle 45))
  (pad "6" smd rect (at 0.325 1.636) (size 0.45 1) (layers "B.Cu" "B.Paste" "B.Mask") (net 8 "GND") (thermal_bridge_angle 45))
  (pad "7" smd rect (at -0.325 1.636) (size 0.45 1) (layers "B.Cu" "B.Paste" "B.Mask") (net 8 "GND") (thermal_bridge_angle 45))
  (pad "8" smd rect (at -0.975 1.636) (size 0.45 1) (layers "B.Cu" "B.Paste" "B.Mask") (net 38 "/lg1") (thermal_bridge_angle 45))
  (pad "9" smd rect (at 0 0.434) (size 4.45 1.036) (layers "B.Cu" "B.Paste" "B.Mask") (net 39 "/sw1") (thermal_bridge_angle 45))
  (pad "10" smd rect (at 0 -0.587) (size 4.45 0.562) (layers "B.Cu" "B.Paste" "B.Mask") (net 41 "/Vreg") (thermal_bridge_angle 45)))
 (segment (start 156.822104 60.634) (end 157.556104 59.9) (width 0.25) (layer "B.Cu") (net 39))
 (segment (start 157.556104 59.9) (end 158.1425 59.9) (width 0.25) (layer "B.Cu") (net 39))
 (segment (start 154.5925 60.634) (end 156.822104 60.634) (width 0.25) (layer "B.Cu") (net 39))
 (segment (start 153.6925 57.764) (end 153.6175 57.839) (width 0.25) (layer "B.Cu") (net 40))
 (segment (start 156.1565 57.764) (end 153.6925 57.764) (width 0.25) (layer "B.Cu") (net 40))
 (segment (start 153.6175 57.839) (end 153.6175 58.564) (width 0.25) (layer "B.Cu") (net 40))
 (segment (start 157.7925 59.4) (end 156.1565 57.764) (width 0.25) (layer "B.Cu") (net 40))
 (segment (start 153.6175 61.836) (end 153.6175 62.586) (width 0.25) (layer "B.Cu") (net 38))
 (segment (start 155.6925 63) (end 157.7925 60.9) (width 0.25) (layer "B.Cu") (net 38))
 (segment (start 154.0315 63) (end 155.6925 63) (width 0.25) (layer "B.Cu") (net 38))
 (segment (start 153.6175 62.586) (end 154.0315 63) (width 0.25) (layer "B.Cu") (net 38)))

